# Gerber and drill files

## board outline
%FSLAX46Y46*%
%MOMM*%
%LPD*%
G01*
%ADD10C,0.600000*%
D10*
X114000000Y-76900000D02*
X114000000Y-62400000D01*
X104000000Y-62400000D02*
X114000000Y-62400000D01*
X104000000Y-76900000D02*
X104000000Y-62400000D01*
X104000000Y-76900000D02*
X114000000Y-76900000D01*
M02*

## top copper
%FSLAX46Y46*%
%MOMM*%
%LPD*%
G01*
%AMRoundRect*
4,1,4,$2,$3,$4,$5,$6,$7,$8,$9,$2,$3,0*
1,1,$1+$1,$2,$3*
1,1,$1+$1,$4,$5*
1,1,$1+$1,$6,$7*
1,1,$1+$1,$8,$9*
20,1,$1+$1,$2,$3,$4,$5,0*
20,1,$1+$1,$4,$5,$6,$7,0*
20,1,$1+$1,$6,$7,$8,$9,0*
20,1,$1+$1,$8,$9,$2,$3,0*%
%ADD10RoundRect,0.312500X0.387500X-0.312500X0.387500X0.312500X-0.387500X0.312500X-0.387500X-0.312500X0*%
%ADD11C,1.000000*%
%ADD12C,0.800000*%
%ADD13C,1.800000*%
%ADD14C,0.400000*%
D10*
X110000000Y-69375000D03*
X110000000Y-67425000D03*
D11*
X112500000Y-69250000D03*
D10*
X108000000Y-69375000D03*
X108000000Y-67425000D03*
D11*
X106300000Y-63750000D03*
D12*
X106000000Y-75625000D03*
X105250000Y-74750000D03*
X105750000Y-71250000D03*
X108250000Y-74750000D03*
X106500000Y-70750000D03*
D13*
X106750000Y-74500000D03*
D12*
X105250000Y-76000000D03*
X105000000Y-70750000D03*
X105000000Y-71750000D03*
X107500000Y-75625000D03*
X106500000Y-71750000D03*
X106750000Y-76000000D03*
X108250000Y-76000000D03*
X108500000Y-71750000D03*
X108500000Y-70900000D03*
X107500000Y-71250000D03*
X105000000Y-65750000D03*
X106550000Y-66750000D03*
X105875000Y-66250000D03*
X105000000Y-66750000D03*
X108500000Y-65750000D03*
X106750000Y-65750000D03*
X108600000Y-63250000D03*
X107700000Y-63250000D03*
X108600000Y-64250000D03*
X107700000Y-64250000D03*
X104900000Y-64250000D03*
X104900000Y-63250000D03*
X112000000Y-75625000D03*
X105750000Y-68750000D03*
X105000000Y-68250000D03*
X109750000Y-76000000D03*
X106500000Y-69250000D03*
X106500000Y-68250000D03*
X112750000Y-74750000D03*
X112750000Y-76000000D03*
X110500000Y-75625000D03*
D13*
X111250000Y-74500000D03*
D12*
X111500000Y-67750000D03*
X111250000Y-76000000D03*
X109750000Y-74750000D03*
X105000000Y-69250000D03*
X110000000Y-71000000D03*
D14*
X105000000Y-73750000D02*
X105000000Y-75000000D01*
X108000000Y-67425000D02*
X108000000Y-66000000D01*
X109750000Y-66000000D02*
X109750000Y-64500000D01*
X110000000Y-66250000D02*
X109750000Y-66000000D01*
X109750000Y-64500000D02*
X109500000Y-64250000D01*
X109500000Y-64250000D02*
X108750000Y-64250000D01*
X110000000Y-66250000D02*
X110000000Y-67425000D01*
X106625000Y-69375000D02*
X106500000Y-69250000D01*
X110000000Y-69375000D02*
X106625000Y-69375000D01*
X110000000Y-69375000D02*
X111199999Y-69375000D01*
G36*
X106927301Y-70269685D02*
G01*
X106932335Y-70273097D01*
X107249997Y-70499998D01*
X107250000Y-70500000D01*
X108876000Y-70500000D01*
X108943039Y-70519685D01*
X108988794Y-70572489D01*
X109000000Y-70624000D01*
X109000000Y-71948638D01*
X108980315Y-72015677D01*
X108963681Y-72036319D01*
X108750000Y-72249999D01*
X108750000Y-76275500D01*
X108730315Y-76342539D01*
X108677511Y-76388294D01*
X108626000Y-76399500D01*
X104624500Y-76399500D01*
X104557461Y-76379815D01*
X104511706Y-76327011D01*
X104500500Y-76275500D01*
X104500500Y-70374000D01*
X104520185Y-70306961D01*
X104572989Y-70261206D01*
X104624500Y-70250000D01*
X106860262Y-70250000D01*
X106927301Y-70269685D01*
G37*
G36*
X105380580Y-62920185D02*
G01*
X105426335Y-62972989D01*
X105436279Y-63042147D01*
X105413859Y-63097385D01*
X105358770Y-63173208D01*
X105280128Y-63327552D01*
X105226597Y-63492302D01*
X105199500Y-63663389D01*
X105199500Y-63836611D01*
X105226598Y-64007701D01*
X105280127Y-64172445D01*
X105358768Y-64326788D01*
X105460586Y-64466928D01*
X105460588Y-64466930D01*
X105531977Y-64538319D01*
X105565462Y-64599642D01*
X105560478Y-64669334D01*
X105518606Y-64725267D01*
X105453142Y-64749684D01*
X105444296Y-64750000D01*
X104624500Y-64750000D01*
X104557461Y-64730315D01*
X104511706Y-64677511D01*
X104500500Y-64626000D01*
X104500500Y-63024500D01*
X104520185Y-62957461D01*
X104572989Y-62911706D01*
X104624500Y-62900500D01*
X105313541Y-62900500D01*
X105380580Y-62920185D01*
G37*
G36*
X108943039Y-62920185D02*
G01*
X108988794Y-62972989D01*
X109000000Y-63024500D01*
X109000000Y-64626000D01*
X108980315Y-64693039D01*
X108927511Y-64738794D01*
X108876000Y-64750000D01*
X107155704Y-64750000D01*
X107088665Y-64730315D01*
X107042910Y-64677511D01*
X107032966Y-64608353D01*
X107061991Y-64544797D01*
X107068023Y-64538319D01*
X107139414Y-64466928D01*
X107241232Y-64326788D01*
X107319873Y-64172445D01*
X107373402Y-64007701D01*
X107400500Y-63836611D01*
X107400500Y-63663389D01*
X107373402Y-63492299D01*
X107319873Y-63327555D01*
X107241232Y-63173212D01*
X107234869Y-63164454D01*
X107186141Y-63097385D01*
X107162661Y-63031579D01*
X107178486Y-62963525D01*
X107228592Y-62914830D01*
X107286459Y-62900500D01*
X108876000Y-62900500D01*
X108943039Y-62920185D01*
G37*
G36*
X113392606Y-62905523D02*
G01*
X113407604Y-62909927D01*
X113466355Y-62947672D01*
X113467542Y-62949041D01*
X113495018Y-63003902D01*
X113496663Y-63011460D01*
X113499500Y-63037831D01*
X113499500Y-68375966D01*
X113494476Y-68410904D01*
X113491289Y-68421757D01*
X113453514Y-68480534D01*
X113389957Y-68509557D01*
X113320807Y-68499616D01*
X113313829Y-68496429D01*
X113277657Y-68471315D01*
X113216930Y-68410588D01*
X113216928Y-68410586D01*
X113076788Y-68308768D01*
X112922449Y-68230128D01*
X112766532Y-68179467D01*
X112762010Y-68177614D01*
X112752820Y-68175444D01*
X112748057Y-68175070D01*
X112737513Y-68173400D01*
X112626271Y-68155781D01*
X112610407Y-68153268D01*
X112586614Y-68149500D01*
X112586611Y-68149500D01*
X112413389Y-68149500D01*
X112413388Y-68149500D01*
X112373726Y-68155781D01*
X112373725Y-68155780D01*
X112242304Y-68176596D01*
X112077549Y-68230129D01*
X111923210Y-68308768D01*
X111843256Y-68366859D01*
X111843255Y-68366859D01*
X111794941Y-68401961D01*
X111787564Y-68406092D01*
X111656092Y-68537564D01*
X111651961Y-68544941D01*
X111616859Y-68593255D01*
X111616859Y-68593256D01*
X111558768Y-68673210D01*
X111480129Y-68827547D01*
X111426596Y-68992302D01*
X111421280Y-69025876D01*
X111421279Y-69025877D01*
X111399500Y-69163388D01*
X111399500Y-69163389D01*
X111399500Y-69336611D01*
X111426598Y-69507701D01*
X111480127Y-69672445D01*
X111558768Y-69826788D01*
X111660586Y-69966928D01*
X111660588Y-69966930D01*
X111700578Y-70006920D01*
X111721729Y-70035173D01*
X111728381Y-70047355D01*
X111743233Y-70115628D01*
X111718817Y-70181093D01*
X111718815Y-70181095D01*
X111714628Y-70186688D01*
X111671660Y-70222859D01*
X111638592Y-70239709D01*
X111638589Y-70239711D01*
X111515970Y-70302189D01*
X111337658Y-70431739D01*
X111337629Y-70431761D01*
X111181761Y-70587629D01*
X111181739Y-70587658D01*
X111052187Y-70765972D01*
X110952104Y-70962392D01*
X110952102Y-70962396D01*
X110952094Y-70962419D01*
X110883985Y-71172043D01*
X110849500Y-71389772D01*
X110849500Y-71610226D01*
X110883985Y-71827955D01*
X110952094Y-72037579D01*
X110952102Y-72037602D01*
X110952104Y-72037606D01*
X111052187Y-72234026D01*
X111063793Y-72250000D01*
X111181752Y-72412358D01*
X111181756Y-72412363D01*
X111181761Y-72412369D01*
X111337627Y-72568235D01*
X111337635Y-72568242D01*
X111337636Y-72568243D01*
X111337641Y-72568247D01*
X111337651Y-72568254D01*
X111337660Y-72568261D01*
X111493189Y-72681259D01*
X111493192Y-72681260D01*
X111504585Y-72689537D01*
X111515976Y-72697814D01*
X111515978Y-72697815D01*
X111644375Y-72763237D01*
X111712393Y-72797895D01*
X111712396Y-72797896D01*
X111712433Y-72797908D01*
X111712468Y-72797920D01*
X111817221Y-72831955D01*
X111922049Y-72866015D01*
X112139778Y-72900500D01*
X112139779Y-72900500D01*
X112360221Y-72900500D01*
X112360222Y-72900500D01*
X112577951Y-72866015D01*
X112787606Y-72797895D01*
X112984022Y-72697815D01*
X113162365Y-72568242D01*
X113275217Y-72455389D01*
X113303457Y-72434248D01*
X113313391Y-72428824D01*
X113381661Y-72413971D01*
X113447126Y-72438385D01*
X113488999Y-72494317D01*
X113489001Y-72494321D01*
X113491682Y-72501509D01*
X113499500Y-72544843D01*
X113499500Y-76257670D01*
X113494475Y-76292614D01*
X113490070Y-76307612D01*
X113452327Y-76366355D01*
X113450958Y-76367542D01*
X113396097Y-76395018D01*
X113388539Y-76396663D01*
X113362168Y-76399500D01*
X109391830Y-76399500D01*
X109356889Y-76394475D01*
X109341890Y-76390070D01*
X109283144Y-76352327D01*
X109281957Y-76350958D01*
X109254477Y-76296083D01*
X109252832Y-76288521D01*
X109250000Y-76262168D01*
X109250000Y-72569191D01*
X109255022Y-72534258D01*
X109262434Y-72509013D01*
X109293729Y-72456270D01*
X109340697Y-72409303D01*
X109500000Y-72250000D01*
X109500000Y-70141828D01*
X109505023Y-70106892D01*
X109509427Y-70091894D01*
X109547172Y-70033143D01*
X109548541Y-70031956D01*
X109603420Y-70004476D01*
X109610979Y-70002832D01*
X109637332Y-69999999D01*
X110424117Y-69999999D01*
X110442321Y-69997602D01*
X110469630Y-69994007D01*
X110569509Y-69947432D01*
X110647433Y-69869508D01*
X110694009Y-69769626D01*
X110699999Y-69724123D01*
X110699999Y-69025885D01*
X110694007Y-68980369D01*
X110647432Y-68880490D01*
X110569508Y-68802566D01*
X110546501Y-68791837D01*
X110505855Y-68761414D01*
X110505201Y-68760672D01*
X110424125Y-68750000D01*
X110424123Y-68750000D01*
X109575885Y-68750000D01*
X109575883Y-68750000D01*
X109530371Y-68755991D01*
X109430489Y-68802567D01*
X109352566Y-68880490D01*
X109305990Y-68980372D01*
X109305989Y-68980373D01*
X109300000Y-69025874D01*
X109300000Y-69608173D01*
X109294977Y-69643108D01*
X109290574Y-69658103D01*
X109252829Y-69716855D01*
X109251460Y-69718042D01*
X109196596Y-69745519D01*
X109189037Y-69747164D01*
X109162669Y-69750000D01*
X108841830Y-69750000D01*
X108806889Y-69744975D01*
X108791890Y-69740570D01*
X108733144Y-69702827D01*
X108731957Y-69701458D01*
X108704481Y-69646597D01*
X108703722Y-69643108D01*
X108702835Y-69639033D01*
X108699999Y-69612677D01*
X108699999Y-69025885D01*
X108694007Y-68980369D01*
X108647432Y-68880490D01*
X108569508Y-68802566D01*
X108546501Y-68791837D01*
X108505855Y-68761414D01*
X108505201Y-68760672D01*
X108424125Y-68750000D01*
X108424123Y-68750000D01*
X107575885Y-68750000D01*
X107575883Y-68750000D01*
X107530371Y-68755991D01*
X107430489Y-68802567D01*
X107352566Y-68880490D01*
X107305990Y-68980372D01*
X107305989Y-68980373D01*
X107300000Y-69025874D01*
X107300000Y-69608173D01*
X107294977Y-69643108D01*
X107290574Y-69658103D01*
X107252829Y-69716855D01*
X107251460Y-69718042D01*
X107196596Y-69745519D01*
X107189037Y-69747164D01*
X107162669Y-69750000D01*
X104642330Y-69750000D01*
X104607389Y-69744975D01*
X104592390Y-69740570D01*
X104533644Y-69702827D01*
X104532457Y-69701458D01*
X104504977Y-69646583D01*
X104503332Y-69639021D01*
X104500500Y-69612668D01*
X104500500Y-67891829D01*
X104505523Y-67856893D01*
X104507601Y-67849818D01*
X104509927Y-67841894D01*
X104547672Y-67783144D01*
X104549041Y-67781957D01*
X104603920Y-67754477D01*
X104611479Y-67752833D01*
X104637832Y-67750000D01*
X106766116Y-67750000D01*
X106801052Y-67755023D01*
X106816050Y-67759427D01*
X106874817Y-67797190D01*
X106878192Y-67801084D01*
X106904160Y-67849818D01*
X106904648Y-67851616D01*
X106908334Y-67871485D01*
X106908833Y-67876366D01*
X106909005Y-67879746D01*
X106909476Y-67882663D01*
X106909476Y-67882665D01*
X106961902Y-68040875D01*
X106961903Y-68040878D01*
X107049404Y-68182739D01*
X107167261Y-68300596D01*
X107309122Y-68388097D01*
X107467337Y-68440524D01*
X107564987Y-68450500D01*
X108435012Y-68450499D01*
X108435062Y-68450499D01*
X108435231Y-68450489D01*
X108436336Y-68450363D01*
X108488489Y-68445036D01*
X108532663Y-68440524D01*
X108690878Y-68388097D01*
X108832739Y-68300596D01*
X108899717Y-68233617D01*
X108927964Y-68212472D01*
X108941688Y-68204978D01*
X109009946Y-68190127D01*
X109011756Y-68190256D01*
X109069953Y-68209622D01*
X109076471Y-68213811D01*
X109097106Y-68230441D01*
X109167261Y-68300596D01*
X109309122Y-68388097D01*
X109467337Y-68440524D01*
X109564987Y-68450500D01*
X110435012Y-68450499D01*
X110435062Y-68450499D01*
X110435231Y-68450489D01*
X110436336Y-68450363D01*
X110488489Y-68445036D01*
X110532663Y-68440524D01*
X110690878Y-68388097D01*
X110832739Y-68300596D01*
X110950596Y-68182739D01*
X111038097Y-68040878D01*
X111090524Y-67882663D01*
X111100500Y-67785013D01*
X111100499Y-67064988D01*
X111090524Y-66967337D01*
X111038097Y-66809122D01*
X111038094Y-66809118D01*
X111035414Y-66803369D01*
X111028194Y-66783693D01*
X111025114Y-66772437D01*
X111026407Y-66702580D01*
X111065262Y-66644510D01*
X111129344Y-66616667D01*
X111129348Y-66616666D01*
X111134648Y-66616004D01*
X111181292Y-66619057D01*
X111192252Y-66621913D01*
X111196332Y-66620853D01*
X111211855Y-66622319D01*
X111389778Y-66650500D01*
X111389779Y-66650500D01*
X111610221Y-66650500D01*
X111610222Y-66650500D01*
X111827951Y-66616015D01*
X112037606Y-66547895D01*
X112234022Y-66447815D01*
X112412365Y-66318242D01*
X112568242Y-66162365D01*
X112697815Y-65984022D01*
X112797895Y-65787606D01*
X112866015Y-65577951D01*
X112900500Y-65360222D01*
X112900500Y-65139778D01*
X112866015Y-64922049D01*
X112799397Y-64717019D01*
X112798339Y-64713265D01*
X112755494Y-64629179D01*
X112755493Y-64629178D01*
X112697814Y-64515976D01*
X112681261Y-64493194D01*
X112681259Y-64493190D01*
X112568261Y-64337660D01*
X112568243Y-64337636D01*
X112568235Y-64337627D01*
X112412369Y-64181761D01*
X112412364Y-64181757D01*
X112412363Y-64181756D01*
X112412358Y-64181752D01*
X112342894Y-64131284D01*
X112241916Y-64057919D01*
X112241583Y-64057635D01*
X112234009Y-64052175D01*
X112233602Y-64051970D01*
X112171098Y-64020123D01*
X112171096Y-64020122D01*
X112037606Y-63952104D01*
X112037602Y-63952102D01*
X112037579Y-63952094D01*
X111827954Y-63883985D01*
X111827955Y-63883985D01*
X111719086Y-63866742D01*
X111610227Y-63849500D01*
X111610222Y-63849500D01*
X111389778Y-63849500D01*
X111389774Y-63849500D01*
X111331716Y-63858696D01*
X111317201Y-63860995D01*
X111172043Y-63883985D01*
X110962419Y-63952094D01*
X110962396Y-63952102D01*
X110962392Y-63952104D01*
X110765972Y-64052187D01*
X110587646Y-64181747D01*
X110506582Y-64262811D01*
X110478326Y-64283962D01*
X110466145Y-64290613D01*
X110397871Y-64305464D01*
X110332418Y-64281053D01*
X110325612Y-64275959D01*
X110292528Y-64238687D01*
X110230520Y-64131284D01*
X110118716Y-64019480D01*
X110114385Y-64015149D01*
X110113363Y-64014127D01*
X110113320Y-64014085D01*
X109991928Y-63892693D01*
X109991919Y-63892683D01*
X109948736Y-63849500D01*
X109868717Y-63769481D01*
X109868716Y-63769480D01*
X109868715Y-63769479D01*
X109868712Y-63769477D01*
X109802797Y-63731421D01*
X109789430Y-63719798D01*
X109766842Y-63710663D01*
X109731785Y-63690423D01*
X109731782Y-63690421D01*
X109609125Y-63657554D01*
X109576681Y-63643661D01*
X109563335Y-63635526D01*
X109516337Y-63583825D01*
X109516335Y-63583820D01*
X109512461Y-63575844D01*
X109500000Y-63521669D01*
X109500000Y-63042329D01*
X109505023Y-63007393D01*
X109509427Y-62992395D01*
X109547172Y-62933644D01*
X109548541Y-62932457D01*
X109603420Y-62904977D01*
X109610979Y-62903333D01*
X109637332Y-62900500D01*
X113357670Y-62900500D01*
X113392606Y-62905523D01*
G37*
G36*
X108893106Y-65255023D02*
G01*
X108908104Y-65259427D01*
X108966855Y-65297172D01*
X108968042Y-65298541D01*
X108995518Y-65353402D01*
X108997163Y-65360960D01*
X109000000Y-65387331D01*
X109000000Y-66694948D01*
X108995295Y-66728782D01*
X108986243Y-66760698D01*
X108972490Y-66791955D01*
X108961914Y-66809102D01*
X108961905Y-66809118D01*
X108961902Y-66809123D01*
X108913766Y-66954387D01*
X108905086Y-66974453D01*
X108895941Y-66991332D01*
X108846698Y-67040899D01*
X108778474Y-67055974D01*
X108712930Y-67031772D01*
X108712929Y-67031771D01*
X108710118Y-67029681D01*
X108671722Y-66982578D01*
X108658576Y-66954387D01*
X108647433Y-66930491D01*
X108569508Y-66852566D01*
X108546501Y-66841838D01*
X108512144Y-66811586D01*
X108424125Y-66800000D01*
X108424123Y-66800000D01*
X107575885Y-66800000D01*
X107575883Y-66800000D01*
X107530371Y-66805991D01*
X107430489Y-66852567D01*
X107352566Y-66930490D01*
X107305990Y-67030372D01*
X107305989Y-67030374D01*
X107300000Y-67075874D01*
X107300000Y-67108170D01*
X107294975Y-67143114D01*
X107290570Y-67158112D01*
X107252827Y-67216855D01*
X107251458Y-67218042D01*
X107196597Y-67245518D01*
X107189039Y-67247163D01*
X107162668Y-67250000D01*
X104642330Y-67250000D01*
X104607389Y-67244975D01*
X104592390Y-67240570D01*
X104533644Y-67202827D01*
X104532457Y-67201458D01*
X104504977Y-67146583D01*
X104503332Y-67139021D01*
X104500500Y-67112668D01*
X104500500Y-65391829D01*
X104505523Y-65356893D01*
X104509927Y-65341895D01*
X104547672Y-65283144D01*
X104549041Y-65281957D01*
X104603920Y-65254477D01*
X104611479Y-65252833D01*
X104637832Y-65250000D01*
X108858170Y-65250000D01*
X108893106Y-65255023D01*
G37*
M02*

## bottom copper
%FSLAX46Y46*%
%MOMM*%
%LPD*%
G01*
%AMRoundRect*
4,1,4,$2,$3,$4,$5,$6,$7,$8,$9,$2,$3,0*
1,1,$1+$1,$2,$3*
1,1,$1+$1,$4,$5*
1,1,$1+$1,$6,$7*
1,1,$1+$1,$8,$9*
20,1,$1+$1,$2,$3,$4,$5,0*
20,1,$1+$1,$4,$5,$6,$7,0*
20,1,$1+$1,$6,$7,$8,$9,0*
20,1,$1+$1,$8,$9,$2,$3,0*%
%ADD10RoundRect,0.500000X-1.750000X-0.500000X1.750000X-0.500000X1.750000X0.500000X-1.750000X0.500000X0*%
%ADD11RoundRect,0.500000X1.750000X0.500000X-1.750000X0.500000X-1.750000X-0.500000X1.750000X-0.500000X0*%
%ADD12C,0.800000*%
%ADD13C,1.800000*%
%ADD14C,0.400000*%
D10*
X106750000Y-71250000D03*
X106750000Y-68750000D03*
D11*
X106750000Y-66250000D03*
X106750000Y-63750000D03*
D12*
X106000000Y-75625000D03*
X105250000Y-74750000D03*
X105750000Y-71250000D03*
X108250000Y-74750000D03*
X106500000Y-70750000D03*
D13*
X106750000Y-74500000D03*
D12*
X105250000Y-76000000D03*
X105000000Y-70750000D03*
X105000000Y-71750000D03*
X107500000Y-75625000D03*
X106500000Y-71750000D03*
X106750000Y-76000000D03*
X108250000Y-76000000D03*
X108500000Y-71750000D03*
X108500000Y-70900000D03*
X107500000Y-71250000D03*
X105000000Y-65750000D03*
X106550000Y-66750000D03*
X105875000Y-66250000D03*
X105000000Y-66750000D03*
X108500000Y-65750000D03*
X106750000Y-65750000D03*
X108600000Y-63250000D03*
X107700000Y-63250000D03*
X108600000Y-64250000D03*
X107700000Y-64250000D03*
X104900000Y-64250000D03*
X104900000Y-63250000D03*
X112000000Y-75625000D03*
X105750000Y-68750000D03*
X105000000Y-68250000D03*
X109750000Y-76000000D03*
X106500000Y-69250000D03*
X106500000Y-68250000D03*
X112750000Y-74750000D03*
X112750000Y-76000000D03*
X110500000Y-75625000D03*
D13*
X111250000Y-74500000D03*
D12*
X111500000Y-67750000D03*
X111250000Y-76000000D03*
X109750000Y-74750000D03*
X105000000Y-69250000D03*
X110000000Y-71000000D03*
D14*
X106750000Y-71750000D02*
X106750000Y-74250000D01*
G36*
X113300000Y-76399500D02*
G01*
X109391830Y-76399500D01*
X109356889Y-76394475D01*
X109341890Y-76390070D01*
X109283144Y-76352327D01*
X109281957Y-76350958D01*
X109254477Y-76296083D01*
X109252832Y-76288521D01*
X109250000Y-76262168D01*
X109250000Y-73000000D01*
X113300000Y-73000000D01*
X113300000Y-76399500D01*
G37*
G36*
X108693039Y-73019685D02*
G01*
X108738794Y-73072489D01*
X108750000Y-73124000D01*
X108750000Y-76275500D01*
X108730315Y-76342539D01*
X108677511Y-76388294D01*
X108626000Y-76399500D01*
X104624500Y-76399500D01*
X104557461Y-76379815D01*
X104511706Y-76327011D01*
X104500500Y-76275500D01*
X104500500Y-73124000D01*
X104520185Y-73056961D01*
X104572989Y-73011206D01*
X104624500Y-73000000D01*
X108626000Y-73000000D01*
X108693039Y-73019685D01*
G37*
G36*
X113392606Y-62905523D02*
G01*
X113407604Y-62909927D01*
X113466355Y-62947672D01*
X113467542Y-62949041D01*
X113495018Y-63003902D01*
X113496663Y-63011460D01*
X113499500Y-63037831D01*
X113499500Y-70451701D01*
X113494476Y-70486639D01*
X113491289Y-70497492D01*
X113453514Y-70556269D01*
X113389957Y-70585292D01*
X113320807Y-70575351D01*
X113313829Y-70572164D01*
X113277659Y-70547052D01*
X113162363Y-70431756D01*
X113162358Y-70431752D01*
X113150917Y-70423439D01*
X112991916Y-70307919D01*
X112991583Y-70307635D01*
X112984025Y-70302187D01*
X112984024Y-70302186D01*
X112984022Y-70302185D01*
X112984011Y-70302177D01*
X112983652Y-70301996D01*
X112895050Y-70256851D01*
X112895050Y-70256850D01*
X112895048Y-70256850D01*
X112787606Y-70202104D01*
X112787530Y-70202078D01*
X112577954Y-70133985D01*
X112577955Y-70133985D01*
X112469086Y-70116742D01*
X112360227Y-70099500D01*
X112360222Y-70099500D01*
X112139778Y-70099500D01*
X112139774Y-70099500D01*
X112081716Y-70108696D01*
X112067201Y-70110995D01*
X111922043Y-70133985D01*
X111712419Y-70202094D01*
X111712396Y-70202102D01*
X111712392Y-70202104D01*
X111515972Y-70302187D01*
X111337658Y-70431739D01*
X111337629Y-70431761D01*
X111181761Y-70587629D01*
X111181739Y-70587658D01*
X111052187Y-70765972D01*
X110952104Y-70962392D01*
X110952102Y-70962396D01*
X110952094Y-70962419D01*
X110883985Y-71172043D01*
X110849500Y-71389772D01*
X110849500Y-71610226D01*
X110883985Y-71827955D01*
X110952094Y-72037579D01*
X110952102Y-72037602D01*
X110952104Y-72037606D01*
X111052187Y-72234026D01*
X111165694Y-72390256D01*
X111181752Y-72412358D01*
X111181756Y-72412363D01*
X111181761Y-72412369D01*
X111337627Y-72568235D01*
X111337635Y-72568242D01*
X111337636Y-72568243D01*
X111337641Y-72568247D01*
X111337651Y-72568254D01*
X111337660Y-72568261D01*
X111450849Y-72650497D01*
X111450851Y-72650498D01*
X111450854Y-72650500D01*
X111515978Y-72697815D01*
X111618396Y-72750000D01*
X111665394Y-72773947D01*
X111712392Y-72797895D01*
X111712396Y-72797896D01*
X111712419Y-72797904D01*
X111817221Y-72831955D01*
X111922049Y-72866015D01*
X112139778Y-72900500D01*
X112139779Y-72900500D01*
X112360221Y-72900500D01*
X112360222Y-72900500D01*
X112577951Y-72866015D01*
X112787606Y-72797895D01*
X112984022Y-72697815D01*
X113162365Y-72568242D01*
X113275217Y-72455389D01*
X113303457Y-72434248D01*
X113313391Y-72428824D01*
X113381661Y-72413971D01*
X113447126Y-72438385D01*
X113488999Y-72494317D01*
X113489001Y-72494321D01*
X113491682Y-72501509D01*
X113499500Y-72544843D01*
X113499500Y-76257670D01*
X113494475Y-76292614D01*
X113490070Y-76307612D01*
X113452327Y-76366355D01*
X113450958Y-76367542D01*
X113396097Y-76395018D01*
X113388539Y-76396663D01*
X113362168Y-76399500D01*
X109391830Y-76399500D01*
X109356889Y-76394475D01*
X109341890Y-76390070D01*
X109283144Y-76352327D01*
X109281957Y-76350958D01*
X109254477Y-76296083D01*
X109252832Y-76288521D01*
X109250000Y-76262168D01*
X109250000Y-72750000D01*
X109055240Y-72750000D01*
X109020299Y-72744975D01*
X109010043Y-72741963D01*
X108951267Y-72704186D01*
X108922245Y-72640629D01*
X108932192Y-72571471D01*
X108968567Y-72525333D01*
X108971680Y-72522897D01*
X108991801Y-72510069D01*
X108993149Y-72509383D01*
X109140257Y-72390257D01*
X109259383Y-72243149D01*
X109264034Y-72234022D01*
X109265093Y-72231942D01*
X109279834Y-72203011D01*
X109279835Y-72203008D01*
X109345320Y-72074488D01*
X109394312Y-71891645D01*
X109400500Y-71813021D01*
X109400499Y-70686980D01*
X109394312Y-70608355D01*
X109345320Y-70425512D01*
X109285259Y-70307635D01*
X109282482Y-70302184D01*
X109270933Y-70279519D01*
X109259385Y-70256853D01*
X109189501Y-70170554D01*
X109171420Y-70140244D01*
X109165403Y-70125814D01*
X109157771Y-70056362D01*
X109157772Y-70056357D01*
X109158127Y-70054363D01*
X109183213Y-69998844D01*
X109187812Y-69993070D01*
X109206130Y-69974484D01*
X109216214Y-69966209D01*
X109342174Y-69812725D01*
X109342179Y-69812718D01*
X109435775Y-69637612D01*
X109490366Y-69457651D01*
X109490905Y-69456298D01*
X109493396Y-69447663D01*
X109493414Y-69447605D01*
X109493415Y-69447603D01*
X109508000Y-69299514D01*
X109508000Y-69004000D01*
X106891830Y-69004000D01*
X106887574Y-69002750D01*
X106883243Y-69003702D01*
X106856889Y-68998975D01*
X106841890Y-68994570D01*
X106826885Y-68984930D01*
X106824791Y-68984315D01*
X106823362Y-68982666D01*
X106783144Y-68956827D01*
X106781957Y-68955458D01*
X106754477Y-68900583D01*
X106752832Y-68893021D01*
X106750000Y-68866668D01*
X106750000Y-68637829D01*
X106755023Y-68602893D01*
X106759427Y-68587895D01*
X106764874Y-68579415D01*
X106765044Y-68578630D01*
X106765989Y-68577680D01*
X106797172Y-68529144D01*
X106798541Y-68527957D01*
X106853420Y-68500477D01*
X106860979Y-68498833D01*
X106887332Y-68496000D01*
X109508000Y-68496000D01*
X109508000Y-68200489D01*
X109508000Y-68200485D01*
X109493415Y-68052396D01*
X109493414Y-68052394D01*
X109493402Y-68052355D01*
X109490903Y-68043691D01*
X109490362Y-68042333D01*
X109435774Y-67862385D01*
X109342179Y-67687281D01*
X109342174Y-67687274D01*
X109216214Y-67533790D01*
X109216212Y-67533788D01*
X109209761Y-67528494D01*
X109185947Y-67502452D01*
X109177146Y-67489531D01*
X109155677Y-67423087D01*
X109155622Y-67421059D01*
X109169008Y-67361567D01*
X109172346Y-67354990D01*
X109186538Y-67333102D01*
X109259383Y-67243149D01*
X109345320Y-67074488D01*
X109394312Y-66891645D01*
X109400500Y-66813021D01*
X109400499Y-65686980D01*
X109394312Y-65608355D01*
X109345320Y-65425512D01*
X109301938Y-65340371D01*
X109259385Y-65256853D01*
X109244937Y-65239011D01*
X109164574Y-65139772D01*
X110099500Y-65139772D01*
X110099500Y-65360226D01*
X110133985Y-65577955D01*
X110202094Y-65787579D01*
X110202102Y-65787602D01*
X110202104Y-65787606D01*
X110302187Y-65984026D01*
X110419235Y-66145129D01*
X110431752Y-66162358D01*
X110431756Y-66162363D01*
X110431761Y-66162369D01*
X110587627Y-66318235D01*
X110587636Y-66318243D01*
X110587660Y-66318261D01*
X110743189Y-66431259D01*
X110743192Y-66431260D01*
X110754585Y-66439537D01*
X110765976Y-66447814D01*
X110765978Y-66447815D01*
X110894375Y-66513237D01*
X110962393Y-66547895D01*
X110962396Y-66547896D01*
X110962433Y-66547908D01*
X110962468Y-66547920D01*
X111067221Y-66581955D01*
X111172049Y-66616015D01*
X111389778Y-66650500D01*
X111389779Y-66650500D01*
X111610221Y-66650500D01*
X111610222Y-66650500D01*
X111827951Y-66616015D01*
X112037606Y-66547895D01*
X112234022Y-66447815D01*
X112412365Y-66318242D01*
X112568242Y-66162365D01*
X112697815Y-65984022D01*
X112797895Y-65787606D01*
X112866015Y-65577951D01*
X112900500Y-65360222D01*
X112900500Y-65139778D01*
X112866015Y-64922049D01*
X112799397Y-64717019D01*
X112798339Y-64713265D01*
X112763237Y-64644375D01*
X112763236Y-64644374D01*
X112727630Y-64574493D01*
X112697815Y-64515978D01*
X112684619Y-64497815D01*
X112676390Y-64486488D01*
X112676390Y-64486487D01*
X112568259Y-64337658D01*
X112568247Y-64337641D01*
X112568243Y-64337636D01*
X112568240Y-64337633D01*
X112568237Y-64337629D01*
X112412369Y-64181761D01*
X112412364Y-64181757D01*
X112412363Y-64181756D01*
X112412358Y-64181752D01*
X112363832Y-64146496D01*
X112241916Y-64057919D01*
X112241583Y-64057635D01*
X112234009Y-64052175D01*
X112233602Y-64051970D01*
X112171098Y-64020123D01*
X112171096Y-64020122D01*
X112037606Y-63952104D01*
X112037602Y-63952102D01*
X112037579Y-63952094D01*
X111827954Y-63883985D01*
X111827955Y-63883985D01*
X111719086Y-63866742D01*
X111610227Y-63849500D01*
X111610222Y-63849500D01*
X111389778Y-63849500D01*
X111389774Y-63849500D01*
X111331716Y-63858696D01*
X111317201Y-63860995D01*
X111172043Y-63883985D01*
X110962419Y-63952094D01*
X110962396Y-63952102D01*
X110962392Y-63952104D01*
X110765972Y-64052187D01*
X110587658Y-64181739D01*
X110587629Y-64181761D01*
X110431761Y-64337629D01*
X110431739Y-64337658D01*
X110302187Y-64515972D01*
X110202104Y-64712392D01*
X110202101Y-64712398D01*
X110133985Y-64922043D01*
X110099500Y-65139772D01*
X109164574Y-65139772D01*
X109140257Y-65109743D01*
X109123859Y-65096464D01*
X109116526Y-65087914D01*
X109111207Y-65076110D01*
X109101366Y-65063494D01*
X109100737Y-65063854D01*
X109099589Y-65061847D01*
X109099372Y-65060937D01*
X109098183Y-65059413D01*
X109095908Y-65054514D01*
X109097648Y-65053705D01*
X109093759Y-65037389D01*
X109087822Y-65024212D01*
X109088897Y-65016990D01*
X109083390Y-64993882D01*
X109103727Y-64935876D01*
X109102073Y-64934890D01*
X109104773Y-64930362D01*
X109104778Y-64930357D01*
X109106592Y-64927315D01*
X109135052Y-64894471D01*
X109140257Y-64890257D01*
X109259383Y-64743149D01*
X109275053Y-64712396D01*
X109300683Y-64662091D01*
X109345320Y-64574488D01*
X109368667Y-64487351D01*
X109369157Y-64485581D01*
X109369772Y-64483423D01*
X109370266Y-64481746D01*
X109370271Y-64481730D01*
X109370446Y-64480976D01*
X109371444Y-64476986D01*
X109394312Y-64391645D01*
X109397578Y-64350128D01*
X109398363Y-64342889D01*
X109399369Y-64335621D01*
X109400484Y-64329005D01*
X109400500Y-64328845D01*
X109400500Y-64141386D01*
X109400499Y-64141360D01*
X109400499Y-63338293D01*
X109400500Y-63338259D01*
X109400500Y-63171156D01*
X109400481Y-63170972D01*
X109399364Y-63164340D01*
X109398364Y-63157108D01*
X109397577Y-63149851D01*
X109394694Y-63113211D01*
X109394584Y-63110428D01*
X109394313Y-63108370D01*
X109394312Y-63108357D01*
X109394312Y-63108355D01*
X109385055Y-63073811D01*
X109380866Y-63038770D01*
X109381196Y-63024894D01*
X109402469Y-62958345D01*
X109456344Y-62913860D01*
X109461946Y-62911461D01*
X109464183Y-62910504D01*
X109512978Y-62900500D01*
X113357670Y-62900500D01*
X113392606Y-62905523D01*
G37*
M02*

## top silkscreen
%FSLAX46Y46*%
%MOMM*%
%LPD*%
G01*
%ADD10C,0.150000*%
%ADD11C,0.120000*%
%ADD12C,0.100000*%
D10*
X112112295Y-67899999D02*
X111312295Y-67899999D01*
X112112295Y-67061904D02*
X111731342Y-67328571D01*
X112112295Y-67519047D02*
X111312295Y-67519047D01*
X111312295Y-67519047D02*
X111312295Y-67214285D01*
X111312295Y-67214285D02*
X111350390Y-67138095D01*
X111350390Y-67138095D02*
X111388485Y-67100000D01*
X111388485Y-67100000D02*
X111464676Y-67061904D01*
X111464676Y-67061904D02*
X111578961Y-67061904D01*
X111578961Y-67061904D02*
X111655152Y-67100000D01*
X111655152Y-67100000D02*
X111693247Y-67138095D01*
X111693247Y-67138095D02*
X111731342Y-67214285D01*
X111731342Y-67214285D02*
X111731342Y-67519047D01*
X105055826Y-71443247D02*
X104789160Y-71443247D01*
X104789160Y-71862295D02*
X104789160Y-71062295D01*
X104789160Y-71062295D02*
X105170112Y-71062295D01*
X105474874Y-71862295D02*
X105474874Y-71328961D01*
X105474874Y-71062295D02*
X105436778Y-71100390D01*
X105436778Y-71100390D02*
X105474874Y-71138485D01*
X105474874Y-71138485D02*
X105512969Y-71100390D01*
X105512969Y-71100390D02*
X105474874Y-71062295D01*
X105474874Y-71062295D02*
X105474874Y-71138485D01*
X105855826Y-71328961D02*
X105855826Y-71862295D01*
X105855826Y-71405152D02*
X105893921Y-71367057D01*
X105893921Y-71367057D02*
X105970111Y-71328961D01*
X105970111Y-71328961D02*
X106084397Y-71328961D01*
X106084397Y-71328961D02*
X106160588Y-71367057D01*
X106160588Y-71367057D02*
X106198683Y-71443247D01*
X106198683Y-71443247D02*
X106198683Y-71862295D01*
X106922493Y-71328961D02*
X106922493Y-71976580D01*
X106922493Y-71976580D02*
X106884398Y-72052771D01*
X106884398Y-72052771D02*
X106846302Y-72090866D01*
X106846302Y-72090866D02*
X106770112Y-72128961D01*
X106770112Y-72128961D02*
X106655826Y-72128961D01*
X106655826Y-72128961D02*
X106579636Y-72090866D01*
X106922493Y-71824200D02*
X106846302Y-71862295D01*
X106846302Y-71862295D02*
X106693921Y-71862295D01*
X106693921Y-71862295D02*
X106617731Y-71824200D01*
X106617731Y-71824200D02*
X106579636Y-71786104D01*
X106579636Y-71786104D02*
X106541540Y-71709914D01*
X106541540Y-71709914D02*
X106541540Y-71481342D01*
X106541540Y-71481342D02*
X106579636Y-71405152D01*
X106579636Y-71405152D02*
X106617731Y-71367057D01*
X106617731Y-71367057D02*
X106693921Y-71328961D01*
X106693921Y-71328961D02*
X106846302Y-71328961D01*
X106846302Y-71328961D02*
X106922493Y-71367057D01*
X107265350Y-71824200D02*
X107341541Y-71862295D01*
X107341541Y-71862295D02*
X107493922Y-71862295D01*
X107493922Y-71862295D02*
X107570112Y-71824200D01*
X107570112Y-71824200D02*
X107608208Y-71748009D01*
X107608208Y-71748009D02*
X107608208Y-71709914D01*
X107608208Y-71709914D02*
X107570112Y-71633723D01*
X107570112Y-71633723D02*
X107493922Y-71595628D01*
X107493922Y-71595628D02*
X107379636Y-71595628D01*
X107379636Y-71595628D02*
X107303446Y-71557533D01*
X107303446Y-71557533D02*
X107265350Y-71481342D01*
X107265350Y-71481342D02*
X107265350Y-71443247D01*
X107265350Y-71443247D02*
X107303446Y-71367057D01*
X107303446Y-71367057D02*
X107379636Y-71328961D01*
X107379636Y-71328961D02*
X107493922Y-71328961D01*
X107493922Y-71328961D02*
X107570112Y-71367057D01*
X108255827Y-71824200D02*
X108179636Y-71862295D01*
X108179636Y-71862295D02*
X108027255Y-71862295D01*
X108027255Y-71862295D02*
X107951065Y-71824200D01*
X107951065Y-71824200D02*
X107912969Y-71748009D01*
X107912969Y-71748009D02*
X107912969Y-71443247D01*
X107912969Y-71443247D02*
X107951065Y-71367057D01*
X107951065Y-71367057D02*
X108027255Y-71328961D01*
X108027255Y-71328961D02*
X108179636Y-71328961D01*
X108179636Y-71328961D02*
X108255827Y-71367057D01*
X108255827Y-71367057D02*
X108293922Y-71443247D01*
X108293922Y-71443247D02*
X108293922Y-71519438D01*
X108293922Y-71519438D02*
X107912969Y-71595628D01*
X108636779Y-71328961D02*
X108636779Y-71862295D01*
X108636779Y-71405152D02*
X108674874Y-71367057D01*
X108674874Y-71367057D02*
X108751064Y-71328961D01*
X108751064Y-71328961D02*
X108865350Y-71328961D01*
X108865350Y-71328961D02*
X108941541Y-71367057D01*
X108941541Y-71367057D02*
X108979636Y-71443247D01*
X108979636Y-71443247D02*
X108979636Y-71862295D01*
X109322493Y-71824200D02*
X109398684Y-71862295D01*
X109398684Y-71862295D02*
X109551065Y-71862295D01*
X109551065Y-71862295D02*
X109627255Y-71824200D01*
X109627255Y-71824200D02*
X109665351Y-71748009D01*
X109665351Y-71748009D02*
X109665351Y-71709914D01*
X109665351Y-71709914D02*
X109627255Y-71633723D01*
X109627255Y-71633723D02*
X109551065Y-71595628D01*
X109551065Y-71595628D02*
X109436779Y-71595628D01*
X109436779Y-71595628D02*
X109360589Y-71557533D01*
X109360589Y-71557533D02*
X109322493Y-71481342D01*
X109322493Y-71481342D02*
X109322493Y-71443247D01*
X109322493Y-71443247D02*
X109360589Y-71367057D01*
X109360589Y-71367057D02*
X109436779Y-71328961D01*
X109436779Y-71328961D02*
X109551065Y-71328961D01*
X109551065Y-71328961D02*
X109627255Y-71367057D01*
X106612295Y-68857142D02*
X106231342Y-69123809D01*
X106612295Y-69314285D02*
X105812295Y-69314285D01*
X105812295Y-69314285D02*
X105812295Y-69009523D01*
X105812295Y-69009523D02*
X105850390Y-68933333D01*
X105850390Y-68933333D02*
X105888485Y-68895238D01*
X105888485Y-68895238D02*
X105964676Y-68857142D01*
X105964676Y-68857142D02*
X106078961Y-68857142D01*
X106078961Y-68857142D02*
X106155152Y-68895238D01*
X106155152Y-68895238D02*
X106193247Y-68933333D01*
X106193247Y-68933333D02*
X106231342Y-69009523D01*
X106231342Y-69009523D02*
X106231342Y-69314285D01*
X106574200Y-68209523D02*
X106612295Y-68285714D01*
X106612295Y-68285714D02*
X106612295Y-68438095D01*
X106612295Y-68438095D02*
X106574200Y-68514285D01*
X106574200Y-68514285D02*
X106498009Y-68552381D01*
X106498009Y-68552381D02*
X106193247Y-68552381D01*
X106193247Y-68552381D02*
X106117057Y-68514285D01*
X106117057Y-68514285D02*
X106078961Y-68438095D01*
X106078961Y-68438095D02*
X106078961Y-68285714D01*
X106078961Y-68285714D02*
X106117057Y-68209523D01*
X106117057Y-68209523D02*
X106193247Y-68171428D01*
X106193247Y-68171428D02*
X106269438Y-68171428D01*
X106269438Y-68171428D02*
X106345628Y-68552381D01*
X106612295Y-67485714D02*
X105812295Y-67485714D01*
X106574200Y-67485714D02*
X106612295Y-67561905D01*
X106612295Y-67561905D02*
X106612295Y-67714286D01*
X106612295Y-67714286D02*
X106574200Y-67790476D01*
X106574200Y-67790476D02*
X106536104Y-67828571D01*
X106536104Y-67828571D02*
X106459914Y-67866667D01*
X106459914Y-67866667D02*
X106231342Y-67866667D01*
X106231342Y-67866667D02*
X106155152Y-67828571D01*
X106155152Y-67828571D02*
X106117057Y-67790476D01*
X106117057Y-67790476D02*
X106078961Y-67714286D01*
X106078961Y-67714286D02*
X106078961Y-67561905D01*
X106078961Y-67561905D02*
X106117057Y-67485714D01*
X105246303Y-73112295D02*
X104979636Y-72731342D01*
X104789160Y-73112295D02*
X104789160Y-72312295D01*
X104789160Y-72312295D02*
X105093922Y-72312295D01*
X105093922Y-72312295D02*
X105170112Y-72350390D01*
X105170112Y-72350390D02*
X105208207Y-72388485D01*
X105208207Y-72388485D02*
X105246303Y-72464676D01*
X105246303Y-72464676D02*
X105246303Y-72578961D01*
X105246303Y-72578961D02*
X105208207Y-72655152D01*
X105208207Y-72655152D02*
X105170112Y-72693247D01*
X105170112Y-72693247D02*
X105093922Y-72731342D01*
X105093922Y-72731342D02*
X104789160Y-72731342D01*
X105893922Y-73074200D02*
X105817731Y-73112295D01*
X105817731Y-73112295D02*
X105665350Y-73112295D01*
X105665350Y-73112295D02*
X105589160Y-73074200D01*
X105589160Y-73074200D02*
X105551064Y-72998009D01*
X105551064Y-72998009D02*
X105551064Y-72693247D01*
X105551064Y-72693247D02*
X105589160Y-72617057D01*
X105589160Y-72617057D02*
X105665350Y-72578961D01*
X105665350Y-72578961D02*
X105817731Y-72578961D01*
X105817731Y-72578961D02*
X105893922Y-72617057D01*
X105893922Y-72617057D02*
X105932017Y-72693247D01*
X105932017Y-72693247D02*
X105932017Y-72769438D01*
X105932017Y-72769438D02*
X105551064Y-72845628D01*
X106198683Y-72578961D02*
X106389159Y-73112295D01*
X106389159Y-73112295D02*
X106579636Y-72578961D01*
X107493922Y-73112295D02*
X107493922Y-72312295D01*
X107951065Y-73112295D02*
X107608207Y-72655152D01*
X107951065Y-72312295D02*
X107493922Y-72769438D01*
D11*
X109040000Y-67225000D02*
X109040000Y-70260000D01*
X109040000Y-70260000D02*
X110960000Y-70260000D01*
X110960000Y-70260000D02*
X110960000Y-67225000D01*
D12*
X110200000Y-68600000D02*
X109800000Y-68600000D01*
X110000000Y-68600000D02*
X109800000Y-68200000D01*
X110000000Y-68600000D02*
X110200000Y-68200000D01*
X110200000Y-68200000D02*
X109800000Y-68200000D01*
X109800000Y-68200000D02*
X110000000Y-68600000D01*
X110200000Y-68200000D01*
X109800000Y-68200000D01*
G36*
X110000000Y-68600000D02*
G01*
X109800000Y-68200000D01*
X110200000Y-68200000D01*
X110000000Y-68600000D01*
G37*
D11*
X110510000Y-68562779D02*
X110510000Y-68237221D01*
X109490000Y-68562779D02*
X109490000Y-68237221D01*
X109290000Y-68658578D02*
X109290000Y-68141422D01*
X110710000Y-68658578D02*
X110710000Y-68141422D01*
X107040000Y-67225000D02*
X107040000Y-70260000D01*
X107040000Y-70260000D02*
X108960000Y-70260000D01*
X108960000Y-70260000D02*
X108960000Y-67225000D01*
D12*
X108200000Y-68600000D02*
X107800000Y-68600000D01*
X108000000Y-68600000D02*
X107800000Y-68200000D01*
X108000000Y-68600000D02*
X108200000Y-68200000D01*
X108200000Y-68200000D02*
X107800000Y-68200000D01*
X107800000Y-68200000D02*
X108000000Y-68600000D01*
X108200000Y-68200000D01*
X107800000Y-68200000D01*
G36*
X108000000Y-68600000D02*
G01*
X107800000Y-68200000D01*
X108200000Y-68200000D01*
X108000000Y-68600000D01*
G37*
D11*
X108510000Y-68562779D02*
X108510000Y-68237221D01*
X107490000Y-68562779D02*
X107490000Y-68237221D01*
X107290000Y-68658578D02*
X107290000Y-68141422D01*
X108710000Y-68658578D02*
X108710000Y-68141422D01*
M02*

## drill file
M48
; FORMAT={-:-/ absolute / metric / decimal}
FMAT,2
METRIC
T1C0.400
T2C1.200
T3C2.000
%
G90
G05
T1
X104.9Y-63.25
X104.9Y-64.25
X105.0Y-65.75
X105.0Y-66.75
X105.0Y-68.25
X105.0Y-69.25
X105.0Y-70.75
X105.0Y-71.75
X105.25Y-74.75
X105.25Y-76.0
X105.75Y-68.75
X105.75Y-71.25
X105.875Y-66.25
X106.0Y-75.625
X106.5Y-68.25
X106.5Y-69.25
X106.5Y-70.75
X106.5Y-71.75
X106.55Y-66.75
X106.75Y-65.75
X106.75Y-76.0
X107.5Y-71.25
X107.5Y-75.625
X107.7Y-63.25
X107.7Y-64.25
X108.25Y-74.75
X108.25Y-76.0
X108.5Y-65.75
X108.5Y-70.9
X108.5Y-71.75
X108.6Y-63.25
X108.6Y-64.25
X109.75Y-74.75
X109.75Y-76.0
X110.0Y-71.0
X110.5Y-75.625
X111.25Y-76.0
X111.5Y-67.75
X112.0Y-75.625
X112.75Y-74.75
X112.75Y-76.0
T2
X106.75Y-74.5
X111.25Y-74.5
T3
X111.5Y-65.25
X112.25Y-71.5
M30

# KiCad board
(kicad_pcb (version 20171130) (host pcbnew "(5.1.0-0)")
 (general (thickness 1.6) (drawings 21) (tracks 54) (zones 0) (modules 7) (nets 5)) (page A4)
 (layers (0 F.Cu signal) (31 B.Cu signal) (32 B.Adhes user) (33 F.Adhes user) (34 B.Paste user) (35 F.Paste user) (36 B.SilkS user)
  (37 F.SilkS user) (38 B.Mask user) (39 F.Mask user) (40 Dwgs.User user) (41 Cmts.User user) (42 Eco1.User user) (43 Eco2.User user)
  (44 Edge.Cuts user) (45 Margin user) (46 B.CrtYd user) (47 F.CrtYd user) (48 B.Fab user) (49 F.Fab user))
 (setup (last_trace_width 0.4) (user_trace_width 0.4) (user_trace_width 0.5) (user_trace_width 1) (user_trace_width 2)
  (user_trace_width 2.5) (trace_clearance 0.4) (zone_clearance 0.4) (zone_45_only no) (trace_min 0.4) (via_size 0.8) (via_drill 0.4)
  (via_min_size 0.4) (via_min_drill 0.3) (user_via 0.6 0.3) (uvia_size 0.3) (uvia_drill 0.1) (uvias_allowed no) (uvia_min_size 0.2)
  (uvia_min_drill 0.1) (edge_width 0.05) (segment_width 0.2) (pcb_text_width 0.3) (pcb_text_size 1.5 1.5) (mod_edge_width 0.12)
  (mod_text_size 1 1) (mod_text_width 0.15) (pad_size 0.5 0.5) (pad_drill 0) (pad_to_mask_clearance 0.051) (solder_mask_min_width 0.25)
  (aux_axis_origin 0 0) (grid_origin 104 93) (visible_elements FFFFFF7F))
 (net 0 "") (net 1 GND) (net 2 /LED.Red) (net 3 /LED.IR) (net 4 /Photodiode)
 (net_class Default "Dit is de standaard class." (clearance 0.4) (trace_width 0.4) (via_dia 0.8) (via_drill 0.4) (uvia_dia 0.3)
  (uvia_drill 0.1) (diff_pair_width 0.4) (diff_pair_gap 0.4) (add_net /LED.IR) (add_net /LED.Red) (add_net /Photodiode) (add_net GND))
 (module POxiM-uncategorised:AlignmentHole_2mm (layer F.Cu) (at 112.25 71.5) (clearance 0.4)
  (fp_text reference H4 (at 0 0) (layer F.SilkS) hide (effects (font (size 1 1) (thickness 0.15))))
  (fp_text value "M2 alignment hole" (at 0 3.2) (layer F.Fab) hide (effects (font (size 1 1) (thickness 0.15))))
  (pad "" np_thru_hole circle (at 0 0) (size 2 2) (drill 2) (layers *.Cu *.Mask)))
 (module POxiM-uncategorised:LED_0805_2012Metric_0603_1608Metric (layer F.Cu) (at 110 68.4 90)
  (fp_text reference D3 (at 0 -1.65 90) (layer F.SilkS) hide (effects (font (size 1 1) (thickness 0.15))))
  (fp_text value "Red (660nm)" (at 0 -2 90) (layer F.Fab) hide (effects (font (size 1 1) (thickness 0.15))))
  (fp_line (start 1.175 -0.96) (end -1.86 -0.96) (layer F.SilkS) (width 0.12))
  (fp_line (start -1.86 -0.96) (end -1.86 0.96) (layer F.SilkS) (width 0.12))
  (fp_line (start -1.86 0.96) (end 1.175 0.96) (layer F.SilkS) (width 0.12))
  (fp_line (start -0.2 0.2) (end -0.2 -0.2) (layer F.SilkS) (width 0.1))
  (fp_line (start -0.2 0) (end 0.2 -0.2) (layer F.SilkS) (width 0.1))
  (fp_line (start -0.2 0) (end 0.2 0.2) (layer F.SilkS) (width 0.1))
  (fp_line (start 0.2 0.2) (end 0.2 -0.2) (layer F.SilkS) (width 0.1))
  (fp_poly (pts (xy 0.2 -0.2) (xy -0.2 0) (xy 0.2 0.2)) (layer F.SilkS) (width 0.1))
  (fp_line (start -0.162779 0.51) (end 0.162779 0.51) (layer F.SilkS) (width 0.12))
  (fp_line (start -0.162779 -0.51) (end 0.162779 -0.51) (layer F.SilkS) (width 0.12))
  (fp_line (start -0.258578 -0.71) (end 0.258578 -0.71) (layer F.SilkS) (width 0.12))
  (fp_line (start -0.258578 0.71) (end 0.258578 0.71) (layer F.SilkS) (width 0.12))
  (pad 1 smd roundrect (at -0.975 0 90) (size 1.25 1.4) (layers F.Cu F.Paste F.Mask) (roundrect_rratio 0.25) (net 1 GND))
  (pad 2 smd roundrect (at 0.975 0 90) (size 1.25 1.4) (layers F.Cu F.Paste F.Mask) (roundrect_rratio 0.25) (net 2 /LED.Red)))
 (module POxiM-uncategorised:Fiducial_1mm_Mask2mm (layer F.Cu) (at 112.5 69.25)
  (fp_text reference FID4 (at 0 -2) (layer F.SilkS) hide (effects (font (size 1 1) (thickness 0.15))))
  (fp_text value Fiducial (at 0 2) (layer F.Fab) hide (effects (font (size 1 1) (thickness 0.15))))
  (pad "" smd circle (at 0 0) (size 1 1) (layers F.Cu F.Mask) (solder_mask_margin 0.5) (clearance 0.6)))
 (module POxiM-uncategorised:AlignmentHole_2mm (layer F.Cu) (at 111.5 65.25) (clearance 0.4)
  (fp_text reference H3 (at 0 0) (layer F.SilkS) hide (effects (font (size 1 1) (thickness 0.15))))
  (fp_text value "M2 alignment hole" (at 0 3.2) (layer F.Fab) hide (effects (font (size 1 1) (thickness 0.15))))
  (pad "" np_thru_hole circle (at 0 0) (size 2 2) (drill 2) (layers *.Cu *.Mask)))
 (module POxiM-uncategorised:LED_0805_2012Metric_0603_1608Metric (layer F.Cu) (at 108 68.4 90)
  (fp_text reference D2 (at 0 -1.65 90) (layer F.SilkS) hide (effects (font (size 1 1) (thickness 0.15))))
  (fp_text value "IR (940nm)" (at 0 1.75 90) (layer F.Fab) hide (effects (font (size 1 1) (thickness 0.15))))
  (fp_line (start 1.175 -0.96) (end -1.86 -0.96) (layer F.SilkS) (width 0.12))
  (fp_line (start -1.86 -0.96) (end -1.86 0.96) (layer F.SilkS) (width 0.12))
  (fp_line (start -1.86 0.96) (end 1.175 0.96) (layer F.SilkS) (width 0.12))
  (fp_line (start -0.2 0.2) (end -0.2 -0.2) (layer F.SilkS) (width 0.1))
  (fp_line (start -0.2 0) (end 0.2 -0.2) (layer F.SilkS) (width 0.1))
  (fp_line (start -0.2 0) (end 0.2 0.2) (layer F.SilkS) (width 0.1))
  (fp_line (start 0.2 0.2) (end 0.2 -0.2) (layer F.SilkS) (width 0.1))
  (fp_poly (pts (xy 0.2 -0.2) (xy -0.2 0) (xy 0.2 0.2)) (layer F.SilkS) (width 0.1))
  (fp_line (start -0.162779 0.51) (end 0.162779 0.51) (layer F.SilkS) (width 0.12))
  (fp_line (start -0.162779 -0.51) (end 0.162779 -0.51) (layer F.SilkS) (width 0.12))
  (fp_line (start -0.258578 -0.71) (end 0.258578 -0.71) (layer F.SilkS) (width 0.12))
  (fp_line (start -0.258578 0.71) (end 0.258578 0.71) (layer F.SilkS) (width 0.12))
  (pad 1 smd roundrect (at -0.975 0 90) (size 1.25 1.4) (layers F.Cu F.Paste F.Mask) (roundrect_rratio 0.25) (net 1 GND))
  (pad 2 smd roundrect (at 0.975 0 90) (size 1.25 1.4) (layers F.Cu F.Paste F.Mask) (roundrect_rratio 0.25) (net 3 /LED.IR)))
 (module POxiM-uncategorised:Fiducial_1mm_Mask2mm (layer F.Cu) (at 106.3 63.75)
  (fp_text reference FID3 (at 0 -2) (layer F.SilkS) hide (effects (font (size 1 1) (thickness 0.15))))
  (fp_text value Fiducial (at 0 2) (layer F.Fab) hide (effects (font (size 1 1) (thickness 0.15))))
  (pad "" smd circle (at 0 0) (size 1 1) (layers F.Cu F.Mask) (solder_mask_margin 0.5) (clearance 0.6)))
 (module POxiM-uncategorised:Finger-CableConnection (layer B.Cu) (at 106.75 67.5 180) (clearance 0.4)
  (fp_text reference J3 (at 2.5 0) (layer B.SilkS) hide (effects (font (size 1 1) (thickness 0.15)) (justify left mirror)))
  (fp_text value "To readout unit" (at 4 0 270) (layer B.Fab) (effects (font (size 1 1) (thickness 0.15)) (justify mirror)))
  (pad 4 smd roundrect (at 0 -3.75) (size 4.5 2) (layers B.Cu B.Mask) (roundrect_rratio 0.25) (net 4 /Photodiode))
  (pad 3 smd roundrect (at 0 -1.25) (size 4.5 2) (layers B.Cu B.Mask) (roundrect_rratio 0.25) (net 1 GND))
  (pad 2 smd roundrect (at 0 1.25 180) (size 4.5 2) (layers B.Cu B.Mask) (roundrect_rratio 0.25) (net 3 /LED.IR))
  (pad 1 smd roundrect (at 0 3.75 180) (size 4.5 2) (layers B.Cu B.Mask) (roundrect_rratio 0.25) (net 2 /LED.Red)))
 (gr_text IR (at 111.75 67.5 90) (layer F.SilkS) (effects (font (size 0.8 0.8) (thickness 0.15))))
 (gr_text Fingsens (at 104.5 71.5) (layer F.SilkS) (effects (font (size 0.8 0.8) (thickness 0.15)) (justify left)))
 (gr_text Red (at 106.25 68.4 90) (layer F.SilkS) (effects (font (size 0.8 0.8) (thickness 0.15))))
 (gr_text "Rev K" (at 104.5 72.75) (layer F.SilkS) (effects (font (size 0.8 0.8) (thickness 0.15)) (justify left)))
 (gr_line (start 114 76.9) (end 114 62.4) (layer Edge.Cuts) (width 0.6))
 (gr_line (start 104 62.4) (end 114 62.4) (layer Edge.Cuts) (width 0.6))
 (gr_line (start 104 76.9) (end 104 62.4) (layer Edge.Cuts) (width 0.6))
 (gr_line (start 104 76.9) (end 114 76.9) (layer Edge.Cuts) (width 0.6))
 (segment (start 106.75 71.75) (end 106.75 74.25) (width 0.4) (layer B.Cu) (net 4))
 (segment (start 105 73.75) (end 105 75) (width 0.4) (layer F.Cu) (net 4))
 (via (at 106 75.625) (size 0.8) (drill 0.4) (layers F.Cu B.Cu) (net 4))
 (via (at 105.25 74.75) (size 0.8) (drill 0.4) (layers F.Cu B.Cu) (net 4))
 (via (at 105.75 71.25) (size 0.8) (drill 0.4) (layers F.Cu B.Cu) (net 4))
 (via (at 108.25 74.75) (size 0.8) (drill 0.4) (layers F.Cu B.Cu) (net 4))
 (via (at 106.5 70.75) (size 0.8) (drill 0.4) (layers F.Cu B.Cu) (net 4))
 (via (at 106.75 74.5) (size 1.8) (drill 1.2) (layers F.Cu B.Cu) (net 4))
 (via (at 105.25 76) (size 0.8) (drill 0.4) (layers F.Cu B.Cu) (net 4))
 (via (at 105 70.75) (size 0.8) (drill 0.4) (layers F.Cu B.Cu) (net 4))
 (via (at 105 71.75) (size 0.8) (drill 0.4) (layers F.Cu B.Cu) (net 4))
 (via (at 107.5 75.625) (size 0.8) (drill 0.4) (layers F.Cu B.Cu) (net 4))
 (via (at 106.5 71.75) (size 0.8) (drill 0.4) (layers F.Cu B.Cu) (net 4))
 (via (at 106.75 76) (size 0.8) (drill 0.4) (layers F.Cu B.Cu) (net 4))
 (via (at 108.25 76) (size 0.8) (drill 0.4) (layers F.Cu B.Cu) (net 4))
 (via (at 108.5 71.75) (size 0.8) (drill 0.4) (layers F.Cu B.Cu) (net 4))
 (via (at 108.5 70.9) (size 0.8) (drill 0.4) (layers F.Cu B.Cu) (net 4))
 (via (at 107.5 71.25) (size 0.8) (drill 0.4) (layers F.Cu B.Cu) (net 4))
 (via (at 105 65.75) (size 0.8) (drill 0.4) (layers F.Cu B.Cu) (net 3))
 (via (at 106.55 66.75) (size 0.8) (drill 0.4) (layers F.Cu B.Cu) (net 3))
 (via (at 105.875 66.25) (size 0.8) (drill 0.4) (layers F.Cu B.Cu) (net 3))
 (via (at 105 66.75) (size 0.8) (drill 0.4) (layers F.Cu B.Cu) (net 3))
 (via (at 108.5 65.75) (size 0.8) (drill 0.4) (layers F.Cu B.Cu) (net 3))
 (via (at 106.75 65.75) (size 0.8) (drill 0.4) (layers F.Cu B.Cu) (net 3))
 (segment (start 108 67.425) (end 108 66) (width 0.4) (layer F.Cu) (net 3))
 (segment (start 109.75 66) (end 109.75 64.5) (width 0.4) (layer F.Cu) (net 2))
 (segment (start 110 66.25) (end 109.75 66) (width 0.4) (layer F.Cu) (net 2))
 (segment (start 109.75 64.5) (end 109.5 64.25) (width 0.4) (layer F.Cu) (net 2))
 (segment (start 109.5 64.25) (end 108.75 64.25) (width 0.4) (layer F.Cu) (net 2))
 (via (at 108.6 63.25) (size 0.8) (drill 0.4) (layers F.Cu B.Cu) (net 2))
 (via (at 107.7 63.25) (size 0.8) (drill 0.4) (layers F.Cu B.Cu) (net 2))
 (via (at 108.6 64.25) (size 0.8) (drill 0.4) (layers F.Cu B.Cu) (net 2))
 (via (at 107.7 64.25) (size 0.8) (drill 0.4) (layers F.Cu B.Cu) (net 2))
 (via (at 104.9 64.25) (size 0.8) (drill 0.4) (layers F.Cu B.Cu) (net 2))
 (via (at 104.9 63.25) (size 0.8) (drill 0.4) (layers F.Cu B.Cu) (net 2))
 (segment (start 110 66.25) (end 110 67.425) (width 0.4) (layer F.Cu) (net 2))
 (via (at 112 75.625) (size 0.8) (drill 0.4) (layers F.Cu B.Cu) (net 1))
 (via (at 105.75 68.75) (size 0.8) (drill 0.4) (layers F.Cu B.Cu) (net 1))
 (via (at 105 68.25) (size 0.8) (drill 0.4) (layers F.Cu B.Cu) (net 1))
 (via (at 109.75 76) (size 0.8) (drill 0.4) (layers F.Cu B.Cu) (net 1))
 (via (at 106.5 69.25) (size 0.8) (drill 0.4) (layers F.Cu B.Cu) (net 1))
 (via (at 106.5 68.25) (size 0.8) (drill 0.4) (layers F.Cu B.Cu) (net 1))
 (via (at 112.75 74.75) (size 0.8) (drill 0.4) (layers F.Cu B.Cu) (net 1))
 (via (at 112.75 76) (size 0.8) (drill 0.4) (layers F.Cu B.Cu) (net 1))
 (via (at 110.5 75.625) (size 0.8) (drill 0.4) (layers F.Cu B.Cu) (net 1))
 (via (at 111.25 74.5) (size 1.8) (drill 1.2) (layers F.Cu B.Cu) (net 1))
 (via (at 111.5 67.75) (size 0.8) (drill 0.4) (layers F.Cu B.Cu) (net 1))
 (via (at 111.25 76) (size 0.8) (drill 0.4) (layers F.Cu B.Cu) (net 1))
 (via (at 109.75 74.75) (size 0.8) (drill 0.4) (layers F.Cu B.Cu) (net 1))
 (via (at 105 69.25) (size 0.8) (drill 0.4) (layers F.Cu B.Cu) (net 1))
 (via (at 110 71) (size 0.8) (drill 0.4) (layers F.Cu B.Cu) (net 1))
 (segment (start 106.625 69.375) (end 106.5 69.25) (width 0.4) (layer F.Cu) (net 1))
 (segment (start 110 69.375) (end 106.625 69.375) (width 0.4) (layer F.Cu) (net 1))
 (segment (start 110 69.375) (end 111.199999 69.375) (width 0.4) (layer F.Cu) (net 1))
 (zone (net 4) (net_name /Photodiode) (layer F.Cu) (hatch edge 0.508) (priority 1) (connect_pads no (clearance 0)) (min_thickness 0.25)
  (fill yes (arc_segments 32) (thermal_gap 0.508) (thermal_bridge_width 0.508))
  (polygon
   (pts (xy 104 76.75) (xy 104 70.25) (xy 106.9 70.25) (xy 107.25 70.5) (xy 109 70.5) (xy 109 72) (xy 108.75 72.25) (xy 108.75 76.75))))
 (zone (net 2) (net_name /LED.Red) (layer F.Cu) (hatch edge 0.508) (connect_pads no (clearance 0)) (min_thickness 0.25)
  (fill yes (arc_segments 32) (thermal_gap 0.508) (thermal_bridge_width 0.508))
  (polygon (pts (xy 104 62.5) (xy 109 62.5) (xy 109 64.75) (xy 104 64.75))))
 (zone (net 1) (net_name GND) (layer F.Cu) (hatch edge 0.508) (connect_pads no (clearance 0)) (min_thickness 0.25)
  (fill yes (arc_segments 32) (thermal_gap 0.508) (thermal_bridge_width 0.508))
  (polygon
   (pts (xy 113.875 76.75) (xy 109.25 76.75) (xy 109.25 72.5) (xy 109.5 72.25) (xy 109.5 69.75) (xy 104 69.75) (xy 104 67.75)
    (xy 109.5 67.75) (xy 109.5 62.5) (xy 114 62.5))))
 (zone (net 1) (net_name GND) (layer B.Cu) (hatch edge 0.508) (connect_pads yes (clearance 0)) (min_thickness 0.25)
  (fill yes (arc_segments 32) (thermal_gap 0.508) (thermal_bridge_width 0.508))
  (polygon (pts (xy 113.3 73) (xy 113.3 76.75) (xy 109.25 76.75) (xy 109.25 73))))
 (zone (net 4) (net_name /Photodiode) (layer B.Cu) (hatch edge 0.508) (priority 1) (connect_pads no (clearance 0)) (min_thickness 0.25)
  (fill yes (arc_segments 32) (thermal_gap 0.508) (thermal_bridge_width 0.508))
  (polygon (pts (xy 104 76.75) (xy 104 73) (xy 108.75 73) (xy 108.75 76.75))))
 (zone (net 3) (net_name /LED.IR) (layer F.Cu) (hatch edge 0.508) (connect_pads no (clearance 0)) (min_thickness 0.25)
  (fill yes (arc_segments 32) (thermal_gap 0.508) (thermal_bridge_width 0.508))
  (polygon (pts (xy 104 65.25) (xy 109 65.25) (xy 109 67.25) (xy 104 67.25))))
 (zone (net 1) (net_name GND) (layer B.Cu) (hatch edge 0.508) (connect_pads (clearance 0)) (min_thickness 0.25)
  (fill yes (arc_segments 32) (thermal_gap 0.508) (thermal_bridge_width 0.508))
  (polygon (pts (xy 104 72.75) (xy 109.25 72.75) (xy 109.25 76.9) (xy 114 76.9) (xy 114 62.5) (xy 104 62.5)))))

